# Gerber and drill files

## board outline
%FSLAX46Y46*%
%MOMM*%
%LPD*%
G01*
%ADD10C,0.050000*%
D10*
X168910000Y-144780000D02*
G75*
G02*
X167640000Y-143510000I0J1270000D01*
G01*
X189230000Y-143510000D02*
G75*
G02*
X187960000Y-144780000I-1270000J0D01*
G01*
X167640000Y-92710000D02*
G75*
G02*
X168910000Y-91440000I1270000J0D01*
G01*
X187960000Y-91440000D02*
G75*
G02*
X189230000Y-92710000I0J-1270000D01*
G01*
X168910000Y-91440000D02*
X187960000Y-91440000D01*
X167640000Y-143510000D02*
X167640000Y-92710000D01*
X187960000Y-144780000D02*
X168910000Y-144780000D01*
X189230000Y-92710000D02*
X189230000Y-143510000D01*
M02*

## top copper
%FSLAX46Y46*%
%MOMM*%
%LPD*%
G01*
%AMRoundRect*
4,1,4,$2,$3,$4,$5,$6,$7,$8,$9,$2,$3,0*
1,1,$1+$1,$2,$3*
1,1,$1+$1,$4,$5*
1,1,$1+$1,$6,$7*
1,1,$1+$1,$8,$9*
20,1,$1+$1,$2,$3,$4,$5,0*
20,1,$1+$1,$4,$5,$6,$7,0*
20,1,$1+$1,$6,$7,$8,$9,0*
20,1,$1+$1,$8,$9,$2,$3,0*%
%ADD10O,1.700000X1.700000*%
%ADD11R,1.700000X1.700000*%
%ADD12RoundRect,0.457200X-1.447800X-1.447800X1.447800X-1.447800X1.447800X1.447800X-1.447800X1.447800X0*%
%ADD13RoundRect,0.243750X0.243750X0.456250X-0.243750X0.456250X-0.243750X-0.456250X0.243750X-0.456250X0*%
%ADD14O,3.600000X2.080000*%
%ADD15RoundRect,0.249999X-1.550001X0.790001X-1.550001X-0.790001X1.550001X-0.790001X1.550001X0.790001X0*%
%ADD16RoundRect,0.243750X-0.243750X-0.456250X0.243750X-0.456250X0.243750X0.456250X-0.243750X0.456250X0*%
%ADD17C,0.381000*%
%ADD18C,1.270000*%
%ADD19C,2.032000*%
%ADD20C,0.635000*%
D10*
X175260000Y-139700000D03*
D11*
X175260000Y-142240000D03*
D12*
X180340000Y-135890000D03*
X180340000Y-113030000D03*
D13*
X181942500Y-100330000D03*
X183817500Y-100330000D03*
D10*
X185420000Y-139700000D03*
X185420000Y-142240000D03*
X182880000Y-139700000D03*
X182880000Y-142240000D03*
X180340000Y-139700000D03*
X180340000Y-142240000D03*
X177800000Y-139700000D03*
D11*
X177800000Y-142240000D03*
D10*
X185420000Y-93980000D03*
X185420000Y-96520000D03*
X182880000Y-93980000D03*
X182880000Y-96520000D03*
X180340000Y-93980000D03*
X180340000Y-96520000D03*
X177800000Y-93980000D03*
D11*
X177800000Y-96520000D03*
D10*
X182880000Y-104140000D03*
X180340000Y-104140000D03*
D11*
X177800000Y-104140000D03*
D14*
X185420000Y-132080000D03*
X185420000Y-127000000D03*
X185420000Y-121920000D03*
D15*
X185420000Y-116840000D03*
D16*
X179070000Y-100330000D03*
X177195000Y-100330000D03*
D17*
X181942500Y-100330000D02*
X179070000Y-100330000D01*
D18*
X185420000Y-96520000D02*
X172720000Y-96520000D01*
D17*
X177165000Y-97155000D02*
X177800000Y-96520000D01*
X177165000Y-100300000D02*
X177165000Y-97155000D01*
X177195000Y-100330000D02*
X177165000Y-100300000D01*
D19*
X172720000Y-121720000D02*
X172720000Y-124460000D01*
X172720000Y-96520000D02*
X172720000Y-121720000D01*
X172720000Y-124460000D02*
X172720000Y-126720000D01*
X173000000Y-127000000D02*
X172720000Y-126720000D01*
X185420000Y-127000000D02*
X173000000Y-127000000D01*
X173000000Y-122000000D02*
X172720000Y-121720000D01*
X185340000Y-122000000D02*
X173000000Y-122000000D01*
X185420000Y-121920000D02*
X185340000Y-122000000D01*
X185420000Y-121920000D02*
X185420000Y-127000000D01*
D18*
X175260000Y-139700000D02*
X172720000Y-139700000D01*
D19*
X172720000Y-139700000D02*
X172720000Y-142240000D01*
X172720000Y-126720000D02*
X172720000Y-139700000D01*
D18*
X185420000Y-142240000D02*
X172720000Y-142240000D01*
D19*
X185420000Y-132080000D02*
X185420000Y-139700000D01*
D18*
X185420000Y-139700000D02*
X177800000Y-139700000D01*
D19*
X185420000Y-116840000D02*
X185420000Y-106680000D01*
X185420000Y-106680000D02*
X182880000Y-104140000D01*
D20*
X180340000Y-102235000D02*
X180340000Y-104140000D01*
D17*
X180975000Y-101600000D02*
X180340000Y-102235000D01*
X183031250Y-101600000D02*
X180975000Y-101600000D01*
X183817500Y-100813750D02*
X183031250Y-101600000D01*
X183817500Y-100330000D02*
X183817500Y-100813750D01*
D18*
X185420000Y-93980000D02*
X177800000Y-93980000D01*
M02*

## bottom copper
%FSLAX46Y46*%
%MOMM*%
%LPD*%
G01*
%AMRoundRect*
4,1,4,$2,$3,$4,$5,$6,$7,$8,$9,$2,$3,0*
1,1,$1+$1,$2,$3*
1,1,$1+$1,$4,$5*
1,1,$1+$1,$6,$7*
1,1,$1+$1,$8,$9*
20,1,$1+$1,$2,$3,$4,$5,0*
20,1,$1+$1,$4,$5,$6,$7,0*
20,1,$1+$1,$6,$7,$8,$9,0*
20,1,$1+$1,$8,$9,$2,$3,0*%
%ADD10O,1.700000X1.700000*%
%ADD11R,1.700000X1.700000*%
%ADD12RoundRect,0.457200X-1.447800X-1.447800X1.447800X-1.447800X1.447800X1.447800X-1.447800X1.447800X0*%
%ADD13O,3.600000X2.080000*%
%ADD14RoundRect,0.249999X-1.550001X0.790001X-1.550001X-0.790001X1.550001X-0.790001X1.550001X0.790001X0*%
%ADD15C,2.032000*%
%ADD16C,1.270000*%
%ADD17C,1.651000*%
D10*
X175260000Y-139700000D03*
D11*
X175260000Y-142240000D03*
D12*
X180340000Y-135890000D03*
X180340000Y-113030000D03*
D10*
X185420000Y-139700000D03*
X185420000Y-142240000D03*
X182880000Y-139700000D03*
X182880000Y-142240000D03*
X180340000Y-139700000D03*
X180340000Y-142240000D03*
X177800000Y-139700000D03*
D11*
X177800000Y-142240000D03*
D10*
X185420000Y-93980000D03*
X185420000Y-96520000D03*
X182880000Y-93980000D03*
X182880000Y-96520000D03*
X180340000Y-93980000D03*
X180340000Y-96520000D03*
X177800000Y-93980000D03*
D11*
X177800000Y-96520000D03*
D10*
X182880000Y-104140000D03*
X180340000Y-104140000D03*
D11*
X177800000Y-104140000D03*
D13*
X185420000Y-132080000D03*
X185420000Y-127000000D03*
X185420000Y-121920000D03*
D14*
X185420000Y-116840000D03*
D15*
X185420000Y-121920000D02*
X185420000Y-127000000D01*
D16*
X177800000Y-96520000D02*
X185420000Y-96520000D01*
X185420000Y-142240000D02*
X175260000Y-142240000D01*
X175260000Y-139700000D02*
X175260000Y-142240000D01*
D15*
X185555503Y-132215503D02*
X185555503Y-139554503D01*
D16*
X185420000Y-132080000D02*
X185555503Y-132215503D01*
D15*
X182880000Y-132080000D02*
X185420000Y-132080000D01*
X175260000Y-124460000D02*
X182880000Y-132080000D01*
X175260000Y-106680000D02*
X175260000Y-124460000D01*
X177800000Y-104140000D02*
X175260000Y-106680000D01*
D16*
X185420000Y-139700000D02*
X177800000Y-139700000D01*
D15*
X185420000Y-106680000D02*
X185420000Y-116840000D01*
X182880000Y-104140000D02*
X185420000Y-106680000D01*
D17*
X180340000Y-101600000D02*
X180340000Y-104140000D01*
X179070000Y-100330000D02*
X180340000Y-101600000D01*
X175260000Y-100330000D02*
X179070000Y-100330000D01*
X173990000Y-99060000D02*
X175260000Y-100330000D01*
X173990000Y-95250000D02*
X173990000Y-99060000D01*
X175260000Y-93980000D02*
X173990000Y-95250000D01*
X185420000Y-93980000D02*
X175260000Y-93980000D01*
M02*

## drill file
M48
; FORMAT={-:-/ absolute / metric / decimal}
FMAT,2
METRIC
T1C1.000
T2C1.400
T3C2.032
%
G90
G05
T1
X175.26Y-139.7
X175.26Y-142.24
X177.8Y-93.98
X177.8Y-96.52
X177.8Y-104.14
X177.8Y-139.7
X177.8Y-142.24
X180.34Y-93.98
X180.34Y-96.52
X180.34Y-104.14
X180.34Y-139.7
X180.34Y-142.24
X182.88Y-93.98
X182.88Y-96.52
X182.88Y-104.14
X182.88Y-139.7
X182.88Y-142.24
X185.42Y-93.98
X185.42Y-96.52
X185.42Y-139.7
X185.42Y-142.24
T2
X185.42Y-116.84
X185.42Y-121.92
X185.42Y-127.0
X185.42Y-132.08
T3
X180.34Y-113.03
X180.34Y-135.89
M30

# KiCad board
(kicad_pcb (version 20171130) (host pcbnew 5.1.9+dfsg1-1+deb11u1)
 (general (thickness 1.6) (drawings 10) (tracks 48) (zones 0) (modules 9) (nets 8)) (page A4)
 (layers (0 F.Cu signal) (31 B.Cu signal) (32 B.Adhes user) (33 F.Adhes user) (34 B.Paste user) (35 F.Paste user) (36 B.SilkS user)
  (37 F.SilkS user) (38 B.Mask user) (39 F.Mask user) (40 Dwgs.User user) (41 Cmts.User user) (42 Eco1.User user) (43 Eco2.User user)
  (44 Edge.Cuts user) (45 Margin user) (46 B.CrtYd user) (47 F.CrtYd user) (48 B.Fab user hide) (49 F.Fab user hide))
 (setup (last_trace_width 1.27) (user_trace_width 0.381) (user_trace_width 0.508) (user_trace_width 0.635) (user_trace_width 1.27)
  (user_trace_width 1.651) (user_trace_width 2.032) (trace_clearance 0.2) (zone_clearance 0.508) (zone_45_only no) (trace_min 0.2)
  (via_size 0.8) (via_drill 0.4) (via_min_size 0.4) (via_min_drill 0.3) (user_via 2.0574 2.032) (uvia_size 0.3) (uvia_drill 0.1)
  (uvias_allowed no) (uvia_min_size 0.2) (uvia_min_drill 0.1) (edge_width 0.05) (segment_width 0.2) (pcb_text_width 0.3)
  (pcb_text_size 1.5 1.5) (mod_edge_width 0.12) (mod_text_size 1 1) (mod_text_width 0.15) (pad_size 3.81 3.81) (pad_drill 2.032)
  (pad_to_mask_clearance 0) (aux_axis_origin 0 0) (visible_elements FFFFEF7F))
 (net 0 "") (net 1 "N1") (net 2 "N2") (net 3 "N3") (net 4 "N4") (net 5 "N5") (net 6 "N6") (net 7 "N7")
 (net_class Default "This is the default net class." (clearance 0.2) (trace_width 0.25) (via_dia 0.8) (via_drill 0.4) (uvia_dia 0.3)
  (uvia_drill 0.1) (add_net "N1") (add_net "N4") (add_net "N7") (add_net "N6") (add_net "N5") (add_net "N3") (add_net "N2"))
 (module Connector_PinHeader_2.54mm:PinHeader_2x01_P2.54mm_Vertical (layer F.Cu) (at 175.26 142.24 90)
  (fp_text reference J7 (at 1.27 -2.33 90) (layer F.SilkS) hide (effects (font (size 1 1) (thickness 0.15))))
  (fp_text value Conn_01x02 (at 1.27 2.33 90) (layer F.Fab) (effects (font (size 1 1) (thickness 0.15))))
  (pad 2 thru_hole oval (at 2.54 0 90) (size 1.7 1.7) (drill 1) (layers *.Cu *.Mask) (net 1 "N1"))
  (pad 1 thru_hole rect (at 0 0 90) (size 1.7 1.7) (drill 1) (layers *.Cu *.Mask) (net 1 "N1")))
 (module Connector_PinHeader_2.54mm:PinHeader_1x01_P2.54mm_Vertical (layer F.Cu) (at 180.34 135.89)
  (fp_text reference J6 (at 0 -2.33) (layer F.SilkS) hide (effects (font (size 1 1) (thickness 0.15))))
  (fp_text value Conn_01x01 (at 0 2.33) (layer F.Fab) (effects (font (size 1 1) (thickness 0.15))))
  (pad 1 thru_hole roundrect (at 0 0) (size 3.81 3.81) (drill 2.032) (layers *.Cu *.Mask) (roundrect_rratio 0.12) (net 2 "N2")))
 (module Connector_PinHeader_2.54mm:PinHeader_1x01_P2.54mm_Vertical (layer F.Cu) (at 180.34 113.03)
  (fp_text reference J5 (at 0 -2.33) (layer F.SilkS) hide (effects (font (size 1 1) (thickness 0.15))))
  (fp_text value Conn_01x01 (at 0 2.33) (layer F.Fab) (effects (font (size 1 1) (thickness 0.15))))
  (pad 1 thru_hole roundrect (at 0 0) (size 3.81 3.81) (drill 2.032) (layers *.Cu *.Mask) (roundrect_rratio 0.12) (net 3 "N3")))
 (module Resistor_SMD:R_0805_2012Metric (layer F.Cu) (at 182.88 100.33 180)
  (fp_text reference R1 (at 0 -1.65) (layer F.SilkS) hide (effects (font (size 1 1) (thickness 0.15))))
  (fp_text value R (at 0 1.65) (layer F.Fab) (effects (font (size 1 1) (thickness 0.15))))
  (pad 2 smd roundrect (at 0.9375 0 180) (size 0.975 1.4) (layers F.Cu F.Paste F.Mask) (roundrect_rratio 0.25) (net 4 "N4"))
  (pad 1 smd roundrect (at -0.9375 0 180) (size 0.975 1.4) (layers F.Cu F.Paste F.Mask) (roundrect_rratio 0.25) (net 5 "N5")))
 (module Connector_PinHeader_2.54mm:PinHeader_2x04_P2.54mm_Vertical (layer F.Cu) (at 177.8 142.24 90)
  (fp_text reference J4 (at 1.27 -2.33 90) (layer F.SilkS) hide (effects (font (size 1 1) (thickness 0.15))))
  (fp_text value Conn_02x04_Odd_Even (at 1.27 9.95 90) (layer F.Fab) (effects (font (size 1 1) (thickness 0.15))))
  (pad 8 thru_hole oval (at 2.54 7.62 90) (size 1.7 1.7) (drill 1) (layers *.Cu *.Mask) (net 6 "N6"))
  (pad 7 thru_hole oval (at 0 7.62 90) (size 1.7 1.7) (drill 1) (layers *.Cu *.Mask) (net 1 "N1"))
  (pad 6 thru_hole oval (at 2.54 5.08 90) (size 1.7 1.7) (drill 1) (layers *.Cu *.Mask) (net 6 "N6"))
  (pad 5 thru_hole oval (at 0 5.08 90) (size 1.7 1.7) (drill 1) (layers *.Cu *.Mask) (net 1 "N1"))
  (pad 4 thru_hole oval (at 2.54 2.54 90) (size 1.7 1.7) (drill 1) (layers *.Cu *.Mask) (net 6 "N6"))
  (pad 3 thru_hole oval (at 0 2.54 90) (size 1.7 1.7) (drill 1) (layers *.Cu *.Mask) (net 1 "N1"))
  (pad 2 thru_hole oval (at 2.54 0 90) (size 1.7 1.7) (drill 1) (layers *.Cu *.Mask) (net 6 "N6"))
  (pad 1 thru_hole rect (at 0 0 90) (size 1.7 1.7) (drill 1) (layers *.Cu *.Mask) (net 1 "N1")))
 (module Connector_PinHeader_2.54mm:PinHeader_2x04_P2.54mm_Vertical (layer F.Cu) (at 177.8 96.52 90)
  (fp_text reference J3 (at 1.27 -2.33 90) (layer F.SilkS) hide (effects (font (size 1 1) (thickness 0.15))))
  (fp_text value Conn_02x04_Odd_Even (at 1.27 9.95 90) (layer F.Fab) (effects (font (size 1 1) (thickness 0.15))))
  (pad 8 thru_hole oval (at 2.54 7.62 90) (size 1.7 1.7) (drill 1) (layers *.Cu *.Mask) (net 5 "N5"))
  (pad 7 thru_hole oval (at 0 7.62 90) (size 1.7 1.7) (drill 1) (layers *.Cu *.Mask) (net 1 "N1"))
  (pad 6 thru_hole oval (at 2.54 5.08 90) (size 1.7 1.7) (drill 1) (layers *.Cu *.Mask) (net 5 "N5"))
  (pad 5 thru_hole oval (at 0 5.08 90) (size 1.7 1.7) (drill 1) (layers *.Cu *.Mask) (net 1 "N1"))
  (pad 4 thru_hole oval (at 2.54 2.54 90) (size 1.7 1.7) (drill 1) (layers *.Cu *.Mask) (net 5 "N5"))
  (pad 3 thru_hole oval (at 0 2.54 90) (size 1.7 1.7) (drill 1) (layers *.Cu *.Mask) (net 1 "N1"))
  (pad 2 thru_hole oval (at 2.54 0 90) (size 1.7 1.7) (drill 1) (layers *.Cu *.Mask) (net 5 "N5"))
  (pad 1 thru_hole rect (at 0 0 90) (size 1.7 1.7) (drill 1) (layers *.Cu *.Mask) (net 1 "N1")))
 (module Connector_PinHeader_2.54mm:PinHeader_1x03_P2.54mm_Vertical (layer F.Cu) (at 177.8 104.14 90)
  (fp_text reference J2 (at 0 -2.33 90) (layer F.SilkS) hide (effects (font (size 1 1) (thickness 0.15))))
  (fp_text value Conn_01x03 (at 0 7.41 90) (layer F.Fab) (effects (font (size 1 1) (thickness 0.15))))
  (pad 3 thru_hole oval (at 0 5.08 90) (size 1.7 1.7) (drill 1) (layers *.Cu *.Mask) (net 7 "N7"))
  (pad 2 thru_hole oval (at 0 2.54 90) (size 1.7 1.7) (drill 1) (layers *.Cu *.Mask) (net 5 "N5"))
  (pad 1 thru_hole rect (at 0 0 90) (size 1.7 1.7) (drill 1) (layers *.Cu *.Mask) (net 6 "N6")))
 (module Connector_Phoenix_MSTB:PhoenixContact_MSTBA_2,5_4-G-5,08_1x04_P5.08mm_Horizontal (layer F.Cu) (at 185.42 116.84 270)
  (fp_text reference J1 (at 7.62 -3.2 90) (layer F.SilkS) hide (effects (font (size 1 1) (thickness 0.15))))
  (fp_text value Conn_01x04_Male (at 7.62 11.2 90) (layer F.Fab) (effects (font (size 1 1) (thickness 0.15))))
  (pad 4 thru_hole oval (at 15.24 0 270) (size 2.08 3.6) (drill 1.4) (layers *.Cu *.Mask) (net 6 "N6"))
  (pad 3 thru_hole oval (at 10.16 0 270) (size 2.08 3.6) (drill 1.4) (layers *.Cu *.Mask) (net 1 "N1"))
  (pad 2 thru_hole oval (at 5.08 0 270) (size 2.08 3.6) (drill 1.4) (layers *.Cu *.Mask) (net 1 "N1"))
  (pad 1 thru_hole roundrect (at 0 0 270) (size 2.08 3.6) (drill 1.4) (layers *.Cu *.Mask) (roundrect_rratio 0.1201918269230769)
   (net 7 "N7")))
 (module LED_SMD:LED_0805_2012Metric (layer F.Cu) (at 178.1325 100.33)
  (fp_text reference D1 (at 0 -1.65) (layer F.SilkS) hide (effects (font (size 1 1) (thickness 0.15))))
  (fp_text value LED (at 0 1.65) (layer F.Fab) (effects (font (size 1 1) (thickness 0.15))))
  (pad 2 smd roundrect (at 0.9375 0) (size 0.975 1.4) (layers F.Cu F.Paste F.Mask) (roundrect_rratio 0.25) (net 4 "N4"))
  (pad 1 smd roundrect (at -0.9375 0) (size 0.975 1.4) (layers F.Cu F.Paste F.Mask) (roundrect_rratio 0.25) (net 1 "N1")))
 (gr_arc (start 168.91 143.51) (end 167.64 143.51) (angle -90) (layer Edge.Cuts) (width 0.05))
 (gr_arc (start 187.96 143.51) (end 187.96 144.78) (angle -90) (layer Edge.Cuts) (width 0.05))
 (gr_arc (start 168.91 92.71) (end 168.91 91.44) (angle -90) (layer Edge.Cuts) (width 0.05))
 (gr_arc (start 187.96 92.71) (end 189.23 92.71) (angle -90) (layer Edge.Cuts) (width 0.05))
 (gr_line (start 168.91 91.44) (end 187.96 91.44) (layer Edge.Cuts) (width 0.05))
 (gr_line (start 167.64 143.51) (end 167.64 92.71) (layer Edge.Cuts) (width 0.05))
 (gr_line (start 187.96 144.78) (end 168.91 144.78) (layer Edge.Cuts) (width 0.05))
 (gr_line (start 189.23 92.71) (end 189.23 143.51) (layer Edge.Cuts) (width 0.05))
 (segment (start 181.9425 100.33) (end 179.07 100.33) (width 0.381) (layer F.Cu) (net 4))
 (segment (start 185.42 96.52) (end 172.72 96.52) (width 1.27) (layer F.Cu) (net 1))
 (segment (start 177.165 97.155) (end 177.8 96.52) (width 0.381) (layer F.Cu) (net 1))
 (segment (start 177.165 100.3) (end 177.165 97.155) (width 0.381) (layer F.Cu) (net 1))
 (segment (start 177.195 100.33) (end 177.165 100.3) (width 0.381) (layer F.Cu) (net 1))
 (segment (start 172.72 121.72) (end 172.72 124.46) (width 2.032) (layer F.Cu) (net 1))
 (segment (start 172.72 96.52) (end 172.72 121.72) (width 2.032) (layer F.Cu) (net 1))
 (segment (start 172.72 124.46) (end 172.72 126.72) (width 2.032) (layer F.Cu) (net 1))
 (segment (start 173 127) (end 172.72 126.72) (width 2.032) (layer F.Cu) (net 1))
 (segment (start 185.42 127) (end 173 127) (width 2.032) (layer F.Cu) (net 1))
 (segment (start 173 122) (end 172.72 121.72) (width 2.032) (layer F.Cu) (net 1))
 (segment (start 185.34 122) (end 173 122) (width 2.032) (layer F.Cu) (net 1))
 (segment (start 185.42 121.92) (end 185.34 122) (width 2.032) (layer F.Cu) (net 1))
 (segment (start 185.42 121.92) (end 185.42 127) (width 2.032) (layer F.Cu) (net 1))
 (segment (start 185.42 121.92) (end 185.42 127) (width 2.032) (layer B.Cu) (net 1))
 (segment (start 175.26 139.7) (end 172.72 139.7) (width 1.27) (layer F.Cu) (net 1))
 (segment (start 172.72 139.7) (end 172.72 142.24) (width 2.032) (layer F.Cu) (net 1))
 (segment (start 172.72 126.72) (end 172.72 139.7) (width 2.032) (layer F.Cu) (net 1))
 (segment (start 185.42 142.24) (end 172.72 142.24) (width 1.27) (layer F.Cu) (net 1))
 (segment (start 177.8 96.52) (end 185.42 96.52) (width 1.27) (layer B.Cu) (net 1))
 (segment (start 185.42 142.24) (end 175.26 142.24) (width 1.27) (layer B.Cu) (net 1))
 (segment (start 175.26 139.7) (end 175.26 142.24) (width 1.27) (layer B.Cu) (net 1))
 (segment (start 185.555503 132.215503) (end 185.555503 139.554503) (width 2.032) (layer B.Cu) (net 6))
 (segment (start 185.42 132.08) (end 185.555503 132.215503) (width 1.27) (layer B.Cu) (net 6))
 (segment (start 182.88 132.08) (end 185.42 132.08) (width 2.032) (layer B.Cu) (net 6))
 (segment (start 175.26 124.46) (end 182.88 132.08) (width 2.032) (layer B.Cu) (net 6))
 (segment (start 175.26 106.68) (end 175.26 124.46) (width 2.032) (layer B.Cu) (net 6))
 (segment (start 177.8 104.14) (end 175.26 106.68) (width 2.032) (layer B.Cu) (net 6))
 (segment (start 185.42 139.7) (end 177.8 139.7) (width 1.27) (layer B.Cu) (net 6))
 (segment (start 185.42 132.08) (end 185.42 139.7) (width 2.032) (layer F.Cu) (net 6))
 (segment (start 185.42 139.7) (end 177.8 139.7) (width 1.27) (layer F.Cu) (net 6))
 (segment (start 185.42 106.68) (end 185.42 116.84) (width 2.032) (layer B.Cu) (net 7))
 (segment (start 182.88 104.14) (end 185.42 106.68) (width 2.032) (layer B.Cu) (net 7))
 (segment (start 185.42 116.84) (end 185.42 106.68) (width 2.032) (layer F.Cu) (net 7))
 (segment (start 185.42 106.68) (end 182.88 104.14) (width 2.032) (layer F.Cu) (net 7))
 (segment (start 180.34 102.235) (end 180.34 104.14) (width 0.635) (layer F.Cu) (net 5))
 (segment (start 180.975 101.6) (end 180.34 102.235) (width 0.381) (layer F.Cu) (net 5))
 (segment (start 183.03125 101.6) (end 180.975 101.6) (width 0.381) (layer F.Cu) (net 5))
 (segment (start 183.8175 100.81375) (end 183.03125 101.6) (width 0.381) (layer F.Cu) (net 5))
 (segment (start 183.8175 100.33) (end 183.8175 100.81375) (width 0.381) (layer F.Cu) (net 5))
 (segment (start 185.42 93.98) (end 177.8 93.98) (width 1.27) (layer F.Cu) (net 5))
 (segment (start 180.34 101.6) (end 180.34 104.14) (width 1.651) (layer B.Cu) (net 5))
 (segment (start 179.07 100.33) (end 180.34 101.6) (width 1.651) (layer B.Cu) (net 5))
 (segment (start 175.26 100.33) (end 179.07 100.33) (width 1.651) (layer B.Cu) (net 5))
 (segment (start 173.99 99.06) (end 175.26 100.33) (width 1.651) (layer B.Cu) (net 5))
 (segment (start 173.99 95.25) (end 173.99 99.06) (width 1.651) (layer B.Cu) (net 5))
 (segment (start 175.26 93.98) (end 173.99 95.25) (width 1.651) (layer B.Cu) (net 5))
 (segment (start 185.42 93.98) (end 175.26 93.98) (width 1.651) (layer B.Cu) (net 5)))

